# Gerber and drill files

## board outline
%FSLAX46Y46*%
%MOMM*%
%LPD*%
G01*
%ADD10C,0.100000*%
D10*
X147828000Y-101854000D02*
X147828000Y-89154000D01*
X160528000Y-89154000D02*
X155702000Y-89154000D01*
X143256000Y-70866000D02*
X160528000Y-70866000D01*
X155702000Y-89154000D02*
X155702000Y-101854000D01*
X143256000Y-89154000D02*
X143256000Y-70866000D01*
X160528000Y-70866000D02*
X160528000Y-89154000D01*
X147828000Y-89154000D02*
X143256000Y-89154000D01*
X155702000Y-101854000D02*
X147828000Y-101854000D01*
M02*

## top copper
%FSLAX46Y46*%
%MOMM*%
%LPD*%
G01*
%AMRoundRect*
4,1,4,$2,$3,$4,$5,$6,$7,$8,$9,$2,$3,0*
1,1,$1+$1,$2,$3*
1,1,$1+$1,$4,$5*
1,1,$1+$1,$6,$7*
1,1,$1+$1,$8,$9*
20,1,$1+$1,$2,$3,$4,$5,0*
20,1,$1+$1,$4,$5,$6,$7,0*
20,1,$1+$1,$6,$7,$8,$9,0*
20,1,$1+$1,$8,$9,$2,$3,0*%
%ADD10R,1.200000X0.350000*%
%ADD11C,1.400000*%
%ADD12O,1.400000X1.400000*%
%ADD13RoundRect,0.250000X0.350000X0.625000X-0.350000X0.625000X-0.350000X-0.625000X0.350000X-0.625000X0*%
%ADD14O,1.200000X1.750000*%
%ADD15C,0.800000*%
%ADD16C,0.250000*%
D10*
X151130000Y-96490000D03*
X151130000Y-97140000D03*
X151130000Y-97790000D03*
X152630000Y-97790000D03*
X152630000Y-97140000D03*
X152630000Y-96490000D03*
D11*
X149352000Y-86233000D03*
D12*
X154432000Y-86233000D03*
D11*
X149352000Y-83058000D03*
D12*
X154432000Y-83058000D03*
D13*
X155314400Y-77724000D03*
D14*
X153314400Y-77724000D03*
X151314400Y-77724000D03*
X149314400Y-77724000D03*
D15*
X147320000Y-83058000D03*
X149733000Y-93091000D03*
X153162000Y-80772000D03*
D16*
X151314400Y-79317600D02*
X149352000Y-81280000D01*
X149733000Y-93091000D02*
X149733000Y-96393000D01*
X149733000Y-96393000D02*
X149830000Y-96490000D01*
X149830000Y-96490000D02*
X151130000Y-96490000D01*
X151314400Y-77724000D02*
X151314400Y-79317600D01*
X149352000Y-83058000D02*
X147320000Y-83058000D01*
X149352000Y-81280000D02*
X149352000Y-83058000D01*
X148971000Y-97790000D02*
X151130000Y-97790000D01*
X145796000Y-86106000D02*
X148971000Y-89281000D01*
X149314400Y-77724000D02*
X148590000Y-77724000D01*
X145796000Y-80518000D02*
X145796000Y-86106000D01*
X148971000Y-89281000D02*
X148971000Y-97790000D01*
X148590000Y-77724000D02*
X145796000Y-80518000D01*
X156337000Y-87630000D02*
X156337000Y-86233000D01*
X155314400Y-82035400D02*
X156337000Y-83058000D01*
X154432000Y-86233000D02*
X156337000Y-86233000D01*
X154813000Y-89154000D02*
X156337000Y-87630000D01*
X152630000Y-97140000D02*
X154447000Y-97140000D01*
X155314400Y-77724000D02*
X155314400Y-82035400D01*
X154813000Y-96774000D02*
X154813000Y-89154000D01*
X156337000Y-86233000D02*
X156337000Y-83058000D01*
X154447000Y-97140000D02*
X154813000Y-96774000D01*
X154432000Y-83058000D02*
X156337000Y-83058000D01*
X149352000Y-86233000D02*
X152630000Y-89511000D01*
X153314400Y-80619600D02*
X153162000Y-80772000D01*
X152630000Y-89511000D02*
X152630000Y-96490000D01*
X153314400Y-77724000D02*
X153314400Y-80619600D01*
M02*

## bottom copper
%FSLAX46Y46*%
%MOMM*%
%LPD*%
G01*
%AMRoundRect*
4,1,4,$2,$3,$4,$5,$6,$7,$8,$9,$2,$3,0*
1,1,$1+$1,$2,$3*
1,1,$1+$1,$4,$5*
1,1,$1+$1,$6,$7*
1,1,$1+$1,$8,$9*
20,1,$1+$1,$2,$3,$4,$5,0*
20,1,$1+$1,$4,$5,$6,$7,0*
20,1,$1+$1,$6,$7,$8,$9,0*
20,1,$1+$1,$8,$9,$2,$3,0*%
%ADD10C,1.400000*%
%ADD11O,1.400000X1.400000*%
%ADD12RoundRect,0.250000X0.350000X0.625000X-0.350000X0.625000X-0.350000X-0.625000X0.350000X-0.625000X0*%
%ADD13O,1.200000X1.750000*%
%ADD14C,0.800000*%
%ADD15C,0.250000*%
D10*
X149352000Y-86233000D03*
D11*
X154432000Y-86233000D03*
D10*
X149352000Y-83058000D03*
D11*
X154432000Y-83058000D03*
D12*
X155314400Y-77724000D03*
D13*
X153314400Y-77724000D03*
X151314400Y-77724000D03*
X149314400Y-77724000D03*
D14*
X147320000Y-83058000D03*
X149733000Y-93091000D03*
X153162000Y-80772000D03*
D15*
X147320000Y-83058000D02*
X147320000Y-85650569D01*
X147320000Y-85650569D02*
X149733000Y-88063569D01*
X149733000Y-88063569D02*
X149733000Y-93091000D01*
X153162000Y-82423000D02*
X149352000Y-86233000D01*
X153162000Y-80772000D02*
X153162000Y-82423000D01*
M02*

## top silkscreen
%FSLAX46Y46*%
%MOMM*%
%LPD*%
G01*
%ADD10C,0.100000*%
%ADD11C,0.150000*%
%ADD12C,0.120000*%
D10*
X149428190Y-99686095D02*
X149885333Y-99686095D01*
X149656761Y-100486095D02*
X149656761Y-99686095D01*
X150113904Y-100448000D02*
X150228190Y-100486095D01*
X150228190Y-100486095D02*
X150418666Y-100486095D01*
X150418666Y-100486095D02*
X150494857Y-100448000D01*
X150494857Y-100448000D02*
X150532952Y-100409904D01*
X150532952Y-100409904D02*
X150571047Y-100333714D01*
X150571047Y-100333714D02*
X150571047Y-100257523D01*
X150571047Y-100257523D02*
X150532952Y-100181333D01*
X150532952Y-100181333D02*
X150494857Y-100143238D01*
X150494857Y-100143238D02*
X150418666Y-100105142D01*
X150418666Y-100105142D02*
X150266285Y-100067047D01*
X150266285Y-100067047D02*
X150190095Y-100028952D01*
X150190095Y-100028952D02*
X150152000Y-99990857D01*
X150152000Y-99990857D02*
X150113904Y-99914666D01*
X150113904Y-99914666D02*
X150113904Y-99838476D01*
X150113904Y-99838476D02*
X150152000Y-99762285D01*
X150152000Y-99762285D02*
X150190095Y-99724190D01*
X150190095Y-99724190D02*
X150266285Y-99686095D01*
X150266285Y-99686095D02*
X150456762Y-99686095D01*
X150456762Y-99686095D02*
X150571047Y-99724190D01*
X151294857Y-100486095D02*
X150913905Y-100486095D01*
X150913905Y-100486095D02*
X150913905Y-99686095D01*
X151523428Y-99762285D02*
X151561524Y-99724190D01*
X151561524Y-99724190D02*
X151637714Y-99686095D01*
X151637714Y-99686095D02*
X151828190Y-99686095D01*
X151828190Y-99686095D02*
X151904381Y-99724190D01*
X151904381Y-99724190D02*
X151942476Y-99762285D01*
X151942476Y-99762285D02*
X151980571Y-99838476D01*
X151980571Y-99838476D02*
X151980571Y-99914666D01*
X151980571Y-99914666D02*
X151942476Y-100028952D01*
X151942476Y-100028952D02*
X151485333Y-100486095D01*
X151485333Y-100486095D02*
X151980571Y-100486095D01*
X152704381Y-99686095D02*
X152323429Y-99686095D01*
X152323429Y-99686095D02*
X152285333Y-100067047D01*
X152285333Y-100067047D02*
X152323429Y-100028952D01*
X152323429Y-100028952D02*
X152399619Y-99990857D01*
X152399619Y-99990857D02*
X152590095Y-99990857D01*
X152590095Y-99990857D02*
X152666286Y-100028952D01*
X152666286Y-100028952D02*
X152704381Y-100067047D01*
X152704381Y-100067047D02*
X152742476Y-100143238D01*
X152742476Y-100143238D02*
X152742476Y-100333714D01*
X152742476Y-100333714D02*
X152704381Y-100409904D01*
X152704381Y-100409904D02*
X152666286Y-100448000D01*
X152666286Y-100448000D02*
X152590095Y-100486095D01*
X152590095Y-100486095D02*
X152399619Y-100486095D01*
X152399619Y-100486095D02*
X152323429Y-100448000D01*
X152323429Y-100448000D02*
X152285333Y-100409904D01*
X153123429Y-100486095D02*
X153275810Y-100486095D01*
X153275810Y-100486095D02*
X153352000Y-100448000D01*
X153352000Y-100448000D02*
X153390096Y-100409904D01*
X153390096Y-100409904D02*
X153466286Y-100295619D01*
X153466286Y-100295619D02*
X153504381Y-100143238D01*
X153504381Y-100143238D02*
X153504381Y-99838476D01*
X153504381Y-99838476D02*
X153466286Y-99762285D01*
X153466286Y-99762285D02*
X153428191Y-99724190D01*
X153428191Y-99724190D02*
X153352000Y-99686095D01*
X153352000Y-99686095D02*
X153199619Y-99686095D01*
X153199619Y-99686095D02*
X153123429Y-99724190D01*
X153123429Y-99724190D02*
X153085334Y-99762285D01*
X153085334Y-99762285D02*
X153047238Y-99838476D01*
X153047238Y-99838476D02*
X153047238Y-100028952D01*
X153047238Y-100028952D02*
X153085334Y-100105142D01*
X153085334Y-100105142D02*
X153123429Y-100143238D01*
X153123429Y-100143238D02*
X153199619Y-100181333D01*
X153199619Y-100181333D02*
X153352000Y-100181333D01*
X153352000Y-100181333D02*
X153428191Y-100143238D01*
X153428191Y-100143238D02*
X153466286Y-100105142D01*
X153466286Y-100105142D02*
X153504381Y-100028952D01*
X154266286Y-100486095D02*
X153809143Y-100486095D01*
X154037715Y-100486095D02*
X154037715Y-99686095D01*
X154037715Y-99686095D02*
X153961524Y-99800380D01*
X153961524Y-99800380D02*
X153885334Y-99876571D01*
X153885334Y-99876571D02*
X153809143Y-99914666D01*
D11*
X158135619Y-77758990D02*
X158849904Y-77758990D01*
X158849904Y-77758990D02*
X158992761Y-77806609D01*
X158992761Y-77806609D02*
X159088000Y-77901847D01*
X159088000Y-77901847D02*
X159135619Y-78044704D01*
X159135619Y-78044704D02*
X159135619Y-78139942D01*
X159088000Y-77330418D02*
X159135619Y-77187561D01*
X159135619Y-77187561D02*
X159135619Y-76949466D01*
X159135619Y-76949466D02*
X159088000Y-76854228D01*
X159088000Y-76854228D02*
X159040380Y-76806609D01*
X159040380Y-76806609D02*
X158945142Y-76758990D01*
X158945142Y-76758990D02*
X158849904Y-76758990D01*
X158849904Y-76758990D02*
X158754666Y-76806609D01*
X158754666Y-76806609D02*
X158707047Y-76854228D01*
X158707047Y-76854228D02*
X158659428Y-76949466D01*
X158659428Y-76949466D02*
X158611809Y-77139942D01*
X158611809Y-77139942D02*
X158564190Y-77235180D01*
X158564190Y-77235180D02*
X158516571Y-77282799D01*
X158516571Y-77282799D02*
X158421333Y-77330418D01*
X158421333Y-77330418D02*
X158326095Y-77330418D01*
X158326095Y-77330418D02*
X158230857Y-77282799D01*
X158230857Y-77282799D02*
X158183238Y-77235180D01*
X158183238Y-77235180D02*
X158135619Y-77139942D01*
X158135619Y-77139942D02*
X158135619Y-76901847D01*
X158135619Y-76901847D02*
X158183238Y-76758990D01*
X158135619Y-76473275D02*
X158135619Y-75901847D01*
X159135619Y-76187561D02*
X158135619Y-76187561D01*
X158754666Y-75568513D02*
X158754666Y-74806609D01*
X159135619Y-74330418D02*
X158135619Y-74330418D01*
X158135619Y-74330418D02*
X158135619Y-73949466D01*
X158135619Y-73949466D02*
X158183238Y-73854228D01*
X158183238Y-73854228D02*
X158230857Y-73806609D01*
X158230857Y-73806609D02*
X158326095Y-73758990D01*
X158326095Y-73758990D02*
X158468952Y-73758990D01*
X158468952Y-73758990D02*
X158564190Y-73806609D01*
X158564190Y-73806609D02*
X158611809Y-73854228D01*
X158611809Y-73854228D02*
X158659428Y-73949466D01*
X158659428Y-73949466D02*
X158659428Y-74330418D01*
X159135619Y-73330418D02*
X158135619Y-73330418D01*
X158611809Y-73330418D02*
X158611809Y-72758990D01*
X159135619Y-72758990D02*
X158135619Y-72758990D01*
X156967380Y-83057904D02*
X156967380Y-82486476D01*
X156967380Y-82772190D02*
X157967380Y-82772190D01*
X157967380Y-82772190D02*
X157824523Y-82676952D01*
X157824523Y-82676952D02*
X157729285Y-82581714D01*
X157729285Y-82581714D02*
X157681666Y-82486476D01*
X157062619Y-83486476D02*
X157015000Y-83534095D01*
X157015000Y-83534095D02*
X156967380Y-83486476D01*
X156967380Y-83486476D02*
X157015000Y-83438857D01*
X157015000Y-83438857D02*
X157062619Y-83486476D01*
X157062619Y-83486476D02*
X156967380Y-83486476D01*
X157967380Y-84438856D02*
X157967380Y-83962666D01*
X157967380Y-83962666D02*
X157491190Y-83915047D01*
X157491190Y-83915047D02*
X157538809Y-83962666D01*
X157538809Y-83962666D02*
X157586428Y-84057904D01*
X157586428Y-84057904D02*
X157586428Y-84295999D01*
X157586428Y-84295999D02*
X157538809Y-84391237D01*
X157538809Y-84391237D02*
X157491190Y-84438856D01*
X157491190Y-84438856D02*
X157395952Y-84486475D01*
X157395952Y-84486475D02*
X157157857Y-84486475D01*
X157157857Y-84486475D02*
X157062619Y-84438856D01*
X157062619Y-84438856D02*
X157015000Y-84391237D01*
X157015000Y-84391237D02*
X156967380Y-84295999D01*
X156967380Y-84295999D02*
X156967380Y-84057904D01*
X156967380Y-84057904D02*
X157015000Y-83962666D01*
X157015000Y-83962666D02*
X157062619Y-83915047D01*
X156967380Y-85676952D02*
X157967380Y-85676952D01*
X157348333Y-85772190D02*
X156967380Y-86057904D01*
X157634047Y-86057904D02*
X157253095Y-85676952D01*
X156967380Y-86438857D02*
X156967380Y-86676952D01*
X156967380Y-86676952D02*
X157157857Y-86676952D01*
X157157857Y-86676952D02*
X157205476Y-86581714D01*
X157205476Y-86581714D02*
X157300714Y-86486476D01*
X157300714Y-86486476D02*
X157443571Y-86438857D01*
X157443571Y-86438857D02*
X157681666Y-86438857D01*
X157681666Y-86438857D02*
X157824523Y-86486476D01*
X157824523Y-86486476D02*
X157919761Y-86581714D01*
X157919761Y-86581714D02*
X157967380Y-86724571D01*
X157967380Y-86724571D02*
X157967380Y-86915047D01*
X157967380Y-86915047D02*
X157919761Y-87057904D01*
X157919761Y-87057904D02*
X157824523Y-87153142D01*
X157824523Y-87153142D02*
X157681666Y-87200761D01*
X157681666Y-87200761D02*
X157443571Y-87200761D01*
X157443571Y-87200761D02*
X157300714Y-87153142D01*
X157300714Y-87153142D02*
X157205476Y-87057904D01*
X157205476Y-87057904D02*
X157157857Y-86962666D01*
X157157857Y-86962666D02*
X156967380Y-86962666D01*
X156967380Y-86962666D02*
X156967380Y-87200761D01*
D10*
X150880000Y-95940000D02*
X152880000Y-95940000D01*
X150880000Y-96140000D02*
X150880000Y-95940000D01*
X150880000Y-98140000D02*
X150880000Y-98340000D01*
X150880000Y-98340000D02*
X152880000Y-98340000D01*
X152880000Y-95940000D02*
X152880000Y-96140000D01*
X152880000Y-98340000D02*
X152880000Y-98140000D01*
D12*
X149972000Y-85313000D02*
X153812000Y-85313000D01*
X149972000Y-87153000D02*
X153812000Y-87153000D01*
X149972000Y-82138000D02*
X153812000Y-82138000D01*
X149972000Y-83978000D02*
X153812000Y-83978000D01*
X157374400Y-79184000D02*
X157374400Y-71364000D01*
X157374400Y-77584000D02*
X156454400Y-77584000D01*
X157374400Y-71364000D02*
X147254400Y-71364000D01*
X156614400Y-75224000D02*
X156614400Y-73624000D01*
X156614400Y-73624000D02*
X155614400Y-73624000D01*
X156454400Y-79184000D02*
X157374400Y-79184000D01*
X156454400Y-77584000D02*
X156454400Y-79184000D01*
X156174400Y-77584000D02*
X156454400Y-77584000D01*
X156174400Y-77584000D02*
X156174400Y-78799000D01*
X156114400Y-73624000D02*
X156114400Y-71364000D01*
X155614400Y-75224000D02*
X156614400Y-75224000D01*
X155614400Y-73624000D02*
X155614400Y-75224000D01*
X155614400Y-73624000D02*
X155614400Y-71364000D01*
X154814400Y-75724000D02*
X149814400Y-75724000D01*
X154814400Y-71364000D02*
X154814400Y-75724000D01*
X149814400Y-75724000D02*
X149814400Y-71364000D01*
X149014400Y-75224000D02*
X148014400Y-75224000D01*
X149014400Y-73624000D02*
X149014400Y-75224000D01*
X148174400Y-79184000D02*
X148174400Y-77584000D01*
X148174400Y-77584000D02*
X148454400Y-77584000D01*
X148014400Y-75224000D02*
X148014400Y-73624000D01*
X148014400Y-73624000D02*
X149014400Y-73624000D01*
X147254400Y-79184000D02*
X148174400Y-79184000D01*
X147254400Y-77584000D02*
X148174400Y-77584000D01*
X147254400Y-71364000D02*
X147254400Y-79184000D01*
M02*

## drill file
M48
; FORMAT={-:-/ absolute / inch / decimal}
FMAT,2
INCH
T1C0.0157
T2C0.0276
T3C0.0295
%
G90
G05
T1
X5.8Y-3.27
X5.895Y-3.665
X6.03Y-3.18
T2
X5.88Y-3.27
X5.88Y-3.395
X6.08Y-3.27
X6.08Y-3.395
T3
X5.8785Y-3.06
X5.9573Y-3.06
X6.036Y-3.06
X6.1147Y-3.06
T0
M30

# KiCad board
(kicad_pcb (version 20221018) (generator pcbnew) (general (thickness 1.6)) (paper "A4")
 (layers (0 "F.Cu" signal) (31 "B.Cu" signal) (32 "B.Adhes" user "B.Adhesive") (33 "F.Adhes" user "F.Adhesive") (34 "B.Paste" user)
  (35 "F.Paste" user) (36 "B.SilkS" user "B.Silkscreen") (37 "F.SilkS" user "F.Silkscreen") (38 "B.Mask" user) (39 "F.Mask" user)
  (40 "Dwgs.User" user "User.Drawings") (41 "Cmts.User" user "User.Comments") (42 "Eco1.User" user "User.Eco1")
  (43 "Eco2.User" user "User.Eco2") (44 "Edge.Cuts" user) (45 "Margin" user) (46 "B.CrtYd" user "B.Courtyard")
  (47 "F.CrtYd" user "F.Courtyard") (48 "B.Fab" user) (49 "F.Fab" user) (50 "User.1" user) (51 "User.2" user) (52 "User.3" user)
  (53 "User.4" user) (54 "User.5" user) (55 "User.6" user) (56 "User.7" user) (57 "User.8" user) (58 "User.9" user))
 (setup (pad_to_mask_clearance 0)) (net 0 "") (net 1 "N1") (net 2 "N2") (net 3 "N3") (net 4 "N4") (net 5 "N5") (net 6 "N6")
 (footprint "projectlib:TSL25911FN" (layer "F.Cu") (at 151.88 97.14)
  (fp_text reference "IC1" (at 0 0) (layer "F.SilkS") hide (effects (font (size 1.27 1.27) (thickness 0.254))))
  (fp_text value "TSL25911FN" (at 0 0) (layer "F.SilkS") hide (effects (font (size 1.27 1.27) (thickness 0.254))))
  (fp_line (start -1 -1.2) (end 1 -1.2) (stroke (width 0.1) (type solid)) (layer "F.SilkS"))
  (fp_line (start -1 -1) (end -1 -1.2) (stroke (width 0.1) (type solid)) (layer "F.SilkS"))
  (fp_line (start -1 1) (end -1 1.2) (stroke (width 0.1) (type solid)) (layer "F.SilkS"))
  (fp_line (start -1 1.2) (end 1 1.2) (stroke (width 0.1) (type solid)) (layer "F.SilkS"))
  (fp_line (start 1 -1.2) (end 1 -1) (stroke (width 0.1) (type solid)) (layer "F.SilkS"))
  (fp_line (start 1 1.2) (end 1 1) (stroke (width 0.1) (type solid)) (layer "F.SilkS"))
  (pad "1" smd rect (at -0.75 -0.65 90) (size 0.35 1.2) (layers "F.Cu" "F.Paste" "F.Mask") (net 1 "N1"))
  (pad "2" smd rect (at -0.75 0 90) (size 0.35 1.2) (layers "F.Cu" "F.Paste" "F.Mask") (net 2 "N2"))
  (pad "3" smd rect (at -0.75 0.65 90) (size 0.35 1.2) (layers "F.Cu" "F.Paste" "F.Mask") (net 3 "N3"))
  (pad "4" smd rect (at 0.75 0.65 90) (size 0.35 1.2) (layers "F.Cu" "F.Paste" "F.Mask") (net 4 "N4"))
  (pad "5" smd rect (at 0.75 0 90) (size 0.35 1.2) (layers "F.Cu" "F.Paste" "F.Mask") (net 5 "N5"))
  (pad "6" smd rect (at 0.75 -0.65 90) (size 0.35 1.2) (layers "F.Cu" "F.Paste" "F.Mask") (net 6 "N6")))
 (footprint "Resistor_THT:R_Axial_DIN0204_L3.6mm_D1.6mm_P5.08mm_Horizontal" (layer "F.Cu") (at 149.352 86.233)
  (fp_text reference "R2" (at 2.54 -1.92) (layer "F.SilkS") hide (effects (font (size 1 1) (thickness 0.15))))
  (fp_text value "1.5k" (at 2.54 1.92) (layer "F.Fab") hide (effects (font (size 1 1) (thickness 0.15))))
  (fp_line (start 0.62 -0.92) (end 4.46 -0.92) (stroke (width 0.12) (type solid)) (layer "F.SilkS"))
  (fp_line (start 0.62 0.92) (end 4.46 0.92) (stroke (width 0.12) (type solid)) (layer "F.SilkS"))
  (pad "1" thru_hole circle (at 0 0) (size 1.4 1.4) (drill 0.7) (layers "*.Cu" "*.Mask") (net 6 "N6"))
  (pad "2" thru_hole oval (at 5.08 0) (size 1.4 1.4) (drill 0.7) (layers "*.Cu" "*.Mask") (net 5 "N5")))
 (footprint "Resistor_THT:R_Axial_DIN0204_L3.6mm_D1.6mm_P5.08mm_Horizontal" (layer "F.Cu") (at 149.352 83.058)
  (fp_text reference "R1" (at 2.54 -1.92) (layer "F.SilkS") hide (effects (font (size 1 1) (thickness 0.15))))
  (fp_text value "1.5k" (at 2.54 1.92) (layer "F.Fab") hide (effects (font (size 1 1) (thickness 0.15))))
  (fp_line (start 0.62 -0.92) (end 4.46 -0.92) (stroke (width 0.12) (type solid)) (layer "F.SilkS"))
  (fp_line (start 0.62 0.92) (end 4.46 0.92) (stroke (width 0.12) (type solid)) (layer "F.SilkS"))
  (pad "1" thru_hole circle (at 0 0) (size 1.4 1.4) (drill 0.7) (layers "*.Cu" "*.Mask") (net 1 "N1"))
  (pad "2" thru_hole oval (at 5.08 0) (size 1.4 1.4) (drill 0.7) (layers "*.Cu" "*.Mask") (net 5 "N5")))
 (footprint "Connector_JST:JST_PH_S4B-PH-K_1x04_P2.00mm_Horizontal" (layer "F.Cu") (at 155.3144 77.724 180)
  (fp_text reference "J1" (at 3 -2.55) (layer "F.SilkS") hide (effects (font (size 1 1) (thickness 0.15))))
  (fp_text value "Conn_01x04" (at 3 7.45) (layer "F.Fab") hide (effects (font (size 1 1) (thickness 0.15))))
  (fp_line (start -2.06 -1.46) (end -2.06 6.36) (stroke (width 0.12) (type solid)) (layer "F.SilkS"))
  (fp_line (start -2.06 0.14) (end -1.14 0.14) (stroke (width 0.12) (type solid)) (layer "F.SilkS"))
  (fp_line (start -2.06 6.36) (end 8.06 6.36) (stroke (width 0.12) (type solid)) (layer "F.SilkS"))
  (fp_line (start -1.3 2.5) (end -1.3 4.1) (stroke (width 0.12) (type solid)) (layer "F.SilkS"))
  (fp_line (start -1.3 4.1) (end -0.3 4.1) (stroke (width 0.12) (type solid)) (layer "F.SilkS"))
  (fp_line (start -1.14 -1.46) (end -2.06 -1.46) (stroke (width 0.12) (type solid)) (layer "F.SilkS"))
  (fp_line (start -1.14 0.14) (end -1.14 -1.46) (stroke (width 0.12) (type solid)) (layer "F.SilkS"))
  (fp_line (start -0.86 0.14) (end -1.14 0.14) (stroke (width 0.12) (type solid)) (layer "F.SilkS"))
  (fp_line (start -0.86 0.14) (end -0.86 -1.075) (stroke (width 0.12) (type solid)) (layer "F.SilkS"))
  (fp_line (start -0.8 4.1) (end -0.8 6.36) (stroke (width 0.12) (type solid)) (layer "F.SilkS"))
  (fp_line (start -0.3 2.5) (end -1.3 2.5) (stroke (width 0.12) (type solid)) (layer "F.SilkS"))
  (fp_line (start -0.3 4.1) (end -0.3 2.5) (stroke (width 0.12) (type solid)) (layer "F.SilkS"))
  (fp_line (start -0.3 4.1) (end -0.3 6.36) (stroke (width 0.12) (type solid)) (layer "F.SilkS"))
  (fp_line (start 0.5 2) (end 5.5 2) (stroke (width 0.12) (type solid)) (layer "F.SilkS"))
  (fp_line (start 0.5 6.36) (end 0.5 2) (stroke (width 0.12) (type solid)) (layer "F.SilkS"))
  (fp_line (start 5.5 2) (end 5.5 6.36) (stroke (width 0.12) (type solid)) (layer "F.SilkS"))
  (fp_line (start 6.3 2.5) (end 7.3 2.5) (stroke (width 0.12) (type solid)) (layer "F.SilkS"))
  (fp_line (start 6.3 4.1) (end 6.3 2.5) (stroke (width 0.12) (type solid)) (layer "F.SilkS"))
  (fp_line (start 7.14 -1.46) (end 7.14 0.14) (stroke (width 0.12) (type solid)) (layer "F.SilkS"))
  (fp_line (start 7.14 0.14) (end 6.86 0.14) (stroke (width 0.12) (type solid)) (layer "F.SilkS"))
  (fp_line (start 7.3 2.5) (end 7.3 4.1) (stroke (width 0.12) (type solid)) (layer "F.SilkS"))
  (fp_line (start 7.3 4.1) (end 6.3 4.1) (stroke (width 0.12) (type solid)) (layer "F.SilkS"))
  (fp_line (start 8.06 -1.46) (end 7.14 -1.46) (stroke (width 0.12) (type solid)) (layer "F.SilkS"))
  (fp_line (start 8.06 0.14) (end 7.14 0.14) (stroke (width 0.12) (type solid)) (layer "F.SilkS"))
  (fp_line (start 8.06 6.36) (end 8.06 -1.46) (stroke (width 0.12) (type solid)) (layer "F.SilkS"))
  (pad "1" thru_hole roundrect (at 0 0 180) (size 1.2 1.75) (drill 0.75) (layers "*.Cu" "*.Mask") (roundrect_rratio 0.2083333333)
   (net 5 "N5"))
  (pad "2" thru_hole oval (at 2 0 180) (size 1.2 1.75) (drill 0.75) (layers "*.Cu" "*.Mask") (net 6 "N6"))
  (pad "3" thru_hole oval (at 4 0 180) (size 1.2 1.75) (drill 0.75) (layers "*.Cu" "*.Mask") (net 1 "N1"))
  (pad "4" thru_hole oval (at 6 0 180) (size 1.2 1.75) (drill 0.75) (layers "*.Cu" "*.Mask") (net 3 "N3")))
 (gr_line (start 147.828 101.854) (end 147.828 89.154) (stroke (width 0.1) (type default)) (layer "Edge.Cuts"))
 (gr_line (start 160.528 89.154) (end 155.702 89.154) (stroke (width 0.1) (type default)) (layer "Edge.Cuts"))
 (gr_line (start 143.256 70.866) (end 160.528 70.866) (stroke (width 0.1) (type default)) (layer "Edge.Cuts"))
 (gr_line (start 155.702 89.154) (end 155.702 101.854) (stroke (width 0.1) (type default)) (layer "Edge.Cuts"))
 (gr_line (start 143.256 89.154) (end 143.256 70.866) (stroke (width 0.1) (type default)) (layer "Edge.Cuts"))
 (gr_line (start 160.528 70.866) (end 160.528 89.154) (stroke (width 0.1) (type default)) (layer "Edge.Cuts"))
 (gr_line (start 147.828 89.154) (end 143.256 89.154) (stroke (width 0.1) (type default)) (layer "Edge.Cuts"))
 (gr_line (start 155.702 101.854) (end 147.828 101.854) (stroke (width 0.1) (type default)) (layer "Edge.Cuts"))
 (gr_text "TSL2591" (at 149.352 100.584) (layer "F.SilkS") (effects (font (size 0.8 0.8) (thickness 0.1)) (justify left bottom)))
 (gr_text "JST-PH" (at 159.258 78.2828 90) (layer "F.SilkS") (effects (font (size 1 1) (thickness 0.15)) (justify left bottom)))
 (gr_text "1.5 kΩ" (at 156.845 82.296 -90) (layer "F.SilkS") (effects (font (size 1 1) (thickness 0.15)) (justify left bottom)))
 (segment (start 151.3144 79.3176) (end 149.352 81.28) (width 0.25) (layer "F.Cu") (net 1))
 (segment (start 149.733 93.091) (end 149.733 96.393) (width 0.25) (layer "F.Cu") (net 1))
 (segment (start 149.733 96.393) (end 149.83 96.49) (width 0.25) (layer "F.Cu") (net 1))
 (segment (start 149.83 96.49) (end 151.13 96.49) (width 0.25) (layer "F.Cu") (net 1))
 (segment (start 151.3144 77.724) (end 151.3144 79.3176) (width 0.25) (layer "F.Cu") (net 1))
 (segment (start 149.352 83.058) (end 147.32 83.058) (width 0.25) (layer "F.Cu") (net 1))
 (segment (start 149.352 81.28) (end 149.352 83.058) (width 0.25) (layer "F.Cu") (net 1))
 (via (at 147.32 83.058) (size 0.8) (drill 0.4) (layers "F.Cu" "B.Cu") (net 1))
 (via (at 149.733 93.091) (size 0.8) (drill 0.4) (layers "F.Cu" "B.Cu") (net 1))
 (segment (start 147.32 83.058) (end 147.32 85.650569) (width 0.25) (layer "B.Cu") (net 1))
 (segment (start 147.32 85.650569) (end 149.733 88.063569) (width 0.25) (layer "B.Cu") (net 1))
 (segment (start 149.733 88.063569) (end 149.733 93.091) (width 0.25) (layer "B.Cu") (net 1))
 (segment (start 148.971 97.79) (end 151.13 97.79) (width 0.25) (layer "F.Cu") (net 3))
 (segment (start 145.796 86.106) (end 148.971 89.281) (width 0.25) (layer "F.Cu") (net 3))
 (segment (start 149.3144 77.724) (end 148.59 77.724) (width 0.25) (layer "F.Cu") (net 3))
 (segment (start 145.796 80.518) (end 145.796 86.106) (width 0.25) (layer "F.Cu") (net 3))
 (segment (start 148.971 89.281) (end 148.971 97.79) (width 0.25) (layer "F.Cu") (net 3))
 (segment (start 148.59 77.724) (end 145.796 80.518) (width 0.25) (layer "F.Cu") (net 3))
 (segment (start 156.337 87.63) (end 156.337 86.233) (width 0.25) (layer "F.Cu") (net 5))
 (segment (start 155.3144 82.0354) (end 156.337 83.058) (width 0.25) (layer "F.Cu") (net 5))
 (segment (start 154.432 86.233) (end 156.337 86.233) (width 0.25) (layer "F.Cu") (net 5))
 (segment (start 154.813 89.154) (end 156.337 87.63) (width 0.25) (layer "F.Cu") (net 5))
 (segment (start 152.63 97.14) (end 154.447 97.14) (width 0.25) (layer "F.Cu") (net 5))
 (segment (start 155.3144 77.724) (end 155.3144 82.0354) (width 0.25) (layer "F.Cu") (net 5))
 (segment (start 154.813 96.774) (end 154.813 89.154) (width 0.25) (layer "F.Cu") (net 5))
 (segment (start 156.337 86.233) (end 156.337 83.058) (width 0.25) (layer "F.Cu") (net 5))
 (segment (start 154.447 97.14) (end 154.813 96.774) (width 0.25) (layer "F.Cu") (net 5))
 (segment (start 154.432 83.058) (end 156.337 83.058) (width 0.25) (layer "F.Cu") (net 5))
 (segment (start 149.352 86.233) (end 152.63 89.511) (width 0.25) (layer "F.Cu") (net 6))
 (segment (start 153.3144 80.6196) (end 153.162 80.772) (width 0.25) (layer "F.Cu") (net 6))
 (segment (start 152.63 89.511) (end 152.63 96.49) (width 0.25) (layer "F.Cu") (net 6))
 (segment (start 153.3144 77.724) (end 153.3144 80.6196) (width 0.25) (layer "F.Cu") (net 6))
 (via (at 153.162 80.772) (size 0.8) (drill 0.4) (layers "F.Cu" "B.Cu") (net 6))
 (segment (start 153.162 82.423) (end 149.352 86.233) (width 0.25) (layer "B.Cu") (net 6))
 (segment (start 153.162 80.772) (end 153.162 82.423) (width 0.25) (layer "B.Cu") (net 6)))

